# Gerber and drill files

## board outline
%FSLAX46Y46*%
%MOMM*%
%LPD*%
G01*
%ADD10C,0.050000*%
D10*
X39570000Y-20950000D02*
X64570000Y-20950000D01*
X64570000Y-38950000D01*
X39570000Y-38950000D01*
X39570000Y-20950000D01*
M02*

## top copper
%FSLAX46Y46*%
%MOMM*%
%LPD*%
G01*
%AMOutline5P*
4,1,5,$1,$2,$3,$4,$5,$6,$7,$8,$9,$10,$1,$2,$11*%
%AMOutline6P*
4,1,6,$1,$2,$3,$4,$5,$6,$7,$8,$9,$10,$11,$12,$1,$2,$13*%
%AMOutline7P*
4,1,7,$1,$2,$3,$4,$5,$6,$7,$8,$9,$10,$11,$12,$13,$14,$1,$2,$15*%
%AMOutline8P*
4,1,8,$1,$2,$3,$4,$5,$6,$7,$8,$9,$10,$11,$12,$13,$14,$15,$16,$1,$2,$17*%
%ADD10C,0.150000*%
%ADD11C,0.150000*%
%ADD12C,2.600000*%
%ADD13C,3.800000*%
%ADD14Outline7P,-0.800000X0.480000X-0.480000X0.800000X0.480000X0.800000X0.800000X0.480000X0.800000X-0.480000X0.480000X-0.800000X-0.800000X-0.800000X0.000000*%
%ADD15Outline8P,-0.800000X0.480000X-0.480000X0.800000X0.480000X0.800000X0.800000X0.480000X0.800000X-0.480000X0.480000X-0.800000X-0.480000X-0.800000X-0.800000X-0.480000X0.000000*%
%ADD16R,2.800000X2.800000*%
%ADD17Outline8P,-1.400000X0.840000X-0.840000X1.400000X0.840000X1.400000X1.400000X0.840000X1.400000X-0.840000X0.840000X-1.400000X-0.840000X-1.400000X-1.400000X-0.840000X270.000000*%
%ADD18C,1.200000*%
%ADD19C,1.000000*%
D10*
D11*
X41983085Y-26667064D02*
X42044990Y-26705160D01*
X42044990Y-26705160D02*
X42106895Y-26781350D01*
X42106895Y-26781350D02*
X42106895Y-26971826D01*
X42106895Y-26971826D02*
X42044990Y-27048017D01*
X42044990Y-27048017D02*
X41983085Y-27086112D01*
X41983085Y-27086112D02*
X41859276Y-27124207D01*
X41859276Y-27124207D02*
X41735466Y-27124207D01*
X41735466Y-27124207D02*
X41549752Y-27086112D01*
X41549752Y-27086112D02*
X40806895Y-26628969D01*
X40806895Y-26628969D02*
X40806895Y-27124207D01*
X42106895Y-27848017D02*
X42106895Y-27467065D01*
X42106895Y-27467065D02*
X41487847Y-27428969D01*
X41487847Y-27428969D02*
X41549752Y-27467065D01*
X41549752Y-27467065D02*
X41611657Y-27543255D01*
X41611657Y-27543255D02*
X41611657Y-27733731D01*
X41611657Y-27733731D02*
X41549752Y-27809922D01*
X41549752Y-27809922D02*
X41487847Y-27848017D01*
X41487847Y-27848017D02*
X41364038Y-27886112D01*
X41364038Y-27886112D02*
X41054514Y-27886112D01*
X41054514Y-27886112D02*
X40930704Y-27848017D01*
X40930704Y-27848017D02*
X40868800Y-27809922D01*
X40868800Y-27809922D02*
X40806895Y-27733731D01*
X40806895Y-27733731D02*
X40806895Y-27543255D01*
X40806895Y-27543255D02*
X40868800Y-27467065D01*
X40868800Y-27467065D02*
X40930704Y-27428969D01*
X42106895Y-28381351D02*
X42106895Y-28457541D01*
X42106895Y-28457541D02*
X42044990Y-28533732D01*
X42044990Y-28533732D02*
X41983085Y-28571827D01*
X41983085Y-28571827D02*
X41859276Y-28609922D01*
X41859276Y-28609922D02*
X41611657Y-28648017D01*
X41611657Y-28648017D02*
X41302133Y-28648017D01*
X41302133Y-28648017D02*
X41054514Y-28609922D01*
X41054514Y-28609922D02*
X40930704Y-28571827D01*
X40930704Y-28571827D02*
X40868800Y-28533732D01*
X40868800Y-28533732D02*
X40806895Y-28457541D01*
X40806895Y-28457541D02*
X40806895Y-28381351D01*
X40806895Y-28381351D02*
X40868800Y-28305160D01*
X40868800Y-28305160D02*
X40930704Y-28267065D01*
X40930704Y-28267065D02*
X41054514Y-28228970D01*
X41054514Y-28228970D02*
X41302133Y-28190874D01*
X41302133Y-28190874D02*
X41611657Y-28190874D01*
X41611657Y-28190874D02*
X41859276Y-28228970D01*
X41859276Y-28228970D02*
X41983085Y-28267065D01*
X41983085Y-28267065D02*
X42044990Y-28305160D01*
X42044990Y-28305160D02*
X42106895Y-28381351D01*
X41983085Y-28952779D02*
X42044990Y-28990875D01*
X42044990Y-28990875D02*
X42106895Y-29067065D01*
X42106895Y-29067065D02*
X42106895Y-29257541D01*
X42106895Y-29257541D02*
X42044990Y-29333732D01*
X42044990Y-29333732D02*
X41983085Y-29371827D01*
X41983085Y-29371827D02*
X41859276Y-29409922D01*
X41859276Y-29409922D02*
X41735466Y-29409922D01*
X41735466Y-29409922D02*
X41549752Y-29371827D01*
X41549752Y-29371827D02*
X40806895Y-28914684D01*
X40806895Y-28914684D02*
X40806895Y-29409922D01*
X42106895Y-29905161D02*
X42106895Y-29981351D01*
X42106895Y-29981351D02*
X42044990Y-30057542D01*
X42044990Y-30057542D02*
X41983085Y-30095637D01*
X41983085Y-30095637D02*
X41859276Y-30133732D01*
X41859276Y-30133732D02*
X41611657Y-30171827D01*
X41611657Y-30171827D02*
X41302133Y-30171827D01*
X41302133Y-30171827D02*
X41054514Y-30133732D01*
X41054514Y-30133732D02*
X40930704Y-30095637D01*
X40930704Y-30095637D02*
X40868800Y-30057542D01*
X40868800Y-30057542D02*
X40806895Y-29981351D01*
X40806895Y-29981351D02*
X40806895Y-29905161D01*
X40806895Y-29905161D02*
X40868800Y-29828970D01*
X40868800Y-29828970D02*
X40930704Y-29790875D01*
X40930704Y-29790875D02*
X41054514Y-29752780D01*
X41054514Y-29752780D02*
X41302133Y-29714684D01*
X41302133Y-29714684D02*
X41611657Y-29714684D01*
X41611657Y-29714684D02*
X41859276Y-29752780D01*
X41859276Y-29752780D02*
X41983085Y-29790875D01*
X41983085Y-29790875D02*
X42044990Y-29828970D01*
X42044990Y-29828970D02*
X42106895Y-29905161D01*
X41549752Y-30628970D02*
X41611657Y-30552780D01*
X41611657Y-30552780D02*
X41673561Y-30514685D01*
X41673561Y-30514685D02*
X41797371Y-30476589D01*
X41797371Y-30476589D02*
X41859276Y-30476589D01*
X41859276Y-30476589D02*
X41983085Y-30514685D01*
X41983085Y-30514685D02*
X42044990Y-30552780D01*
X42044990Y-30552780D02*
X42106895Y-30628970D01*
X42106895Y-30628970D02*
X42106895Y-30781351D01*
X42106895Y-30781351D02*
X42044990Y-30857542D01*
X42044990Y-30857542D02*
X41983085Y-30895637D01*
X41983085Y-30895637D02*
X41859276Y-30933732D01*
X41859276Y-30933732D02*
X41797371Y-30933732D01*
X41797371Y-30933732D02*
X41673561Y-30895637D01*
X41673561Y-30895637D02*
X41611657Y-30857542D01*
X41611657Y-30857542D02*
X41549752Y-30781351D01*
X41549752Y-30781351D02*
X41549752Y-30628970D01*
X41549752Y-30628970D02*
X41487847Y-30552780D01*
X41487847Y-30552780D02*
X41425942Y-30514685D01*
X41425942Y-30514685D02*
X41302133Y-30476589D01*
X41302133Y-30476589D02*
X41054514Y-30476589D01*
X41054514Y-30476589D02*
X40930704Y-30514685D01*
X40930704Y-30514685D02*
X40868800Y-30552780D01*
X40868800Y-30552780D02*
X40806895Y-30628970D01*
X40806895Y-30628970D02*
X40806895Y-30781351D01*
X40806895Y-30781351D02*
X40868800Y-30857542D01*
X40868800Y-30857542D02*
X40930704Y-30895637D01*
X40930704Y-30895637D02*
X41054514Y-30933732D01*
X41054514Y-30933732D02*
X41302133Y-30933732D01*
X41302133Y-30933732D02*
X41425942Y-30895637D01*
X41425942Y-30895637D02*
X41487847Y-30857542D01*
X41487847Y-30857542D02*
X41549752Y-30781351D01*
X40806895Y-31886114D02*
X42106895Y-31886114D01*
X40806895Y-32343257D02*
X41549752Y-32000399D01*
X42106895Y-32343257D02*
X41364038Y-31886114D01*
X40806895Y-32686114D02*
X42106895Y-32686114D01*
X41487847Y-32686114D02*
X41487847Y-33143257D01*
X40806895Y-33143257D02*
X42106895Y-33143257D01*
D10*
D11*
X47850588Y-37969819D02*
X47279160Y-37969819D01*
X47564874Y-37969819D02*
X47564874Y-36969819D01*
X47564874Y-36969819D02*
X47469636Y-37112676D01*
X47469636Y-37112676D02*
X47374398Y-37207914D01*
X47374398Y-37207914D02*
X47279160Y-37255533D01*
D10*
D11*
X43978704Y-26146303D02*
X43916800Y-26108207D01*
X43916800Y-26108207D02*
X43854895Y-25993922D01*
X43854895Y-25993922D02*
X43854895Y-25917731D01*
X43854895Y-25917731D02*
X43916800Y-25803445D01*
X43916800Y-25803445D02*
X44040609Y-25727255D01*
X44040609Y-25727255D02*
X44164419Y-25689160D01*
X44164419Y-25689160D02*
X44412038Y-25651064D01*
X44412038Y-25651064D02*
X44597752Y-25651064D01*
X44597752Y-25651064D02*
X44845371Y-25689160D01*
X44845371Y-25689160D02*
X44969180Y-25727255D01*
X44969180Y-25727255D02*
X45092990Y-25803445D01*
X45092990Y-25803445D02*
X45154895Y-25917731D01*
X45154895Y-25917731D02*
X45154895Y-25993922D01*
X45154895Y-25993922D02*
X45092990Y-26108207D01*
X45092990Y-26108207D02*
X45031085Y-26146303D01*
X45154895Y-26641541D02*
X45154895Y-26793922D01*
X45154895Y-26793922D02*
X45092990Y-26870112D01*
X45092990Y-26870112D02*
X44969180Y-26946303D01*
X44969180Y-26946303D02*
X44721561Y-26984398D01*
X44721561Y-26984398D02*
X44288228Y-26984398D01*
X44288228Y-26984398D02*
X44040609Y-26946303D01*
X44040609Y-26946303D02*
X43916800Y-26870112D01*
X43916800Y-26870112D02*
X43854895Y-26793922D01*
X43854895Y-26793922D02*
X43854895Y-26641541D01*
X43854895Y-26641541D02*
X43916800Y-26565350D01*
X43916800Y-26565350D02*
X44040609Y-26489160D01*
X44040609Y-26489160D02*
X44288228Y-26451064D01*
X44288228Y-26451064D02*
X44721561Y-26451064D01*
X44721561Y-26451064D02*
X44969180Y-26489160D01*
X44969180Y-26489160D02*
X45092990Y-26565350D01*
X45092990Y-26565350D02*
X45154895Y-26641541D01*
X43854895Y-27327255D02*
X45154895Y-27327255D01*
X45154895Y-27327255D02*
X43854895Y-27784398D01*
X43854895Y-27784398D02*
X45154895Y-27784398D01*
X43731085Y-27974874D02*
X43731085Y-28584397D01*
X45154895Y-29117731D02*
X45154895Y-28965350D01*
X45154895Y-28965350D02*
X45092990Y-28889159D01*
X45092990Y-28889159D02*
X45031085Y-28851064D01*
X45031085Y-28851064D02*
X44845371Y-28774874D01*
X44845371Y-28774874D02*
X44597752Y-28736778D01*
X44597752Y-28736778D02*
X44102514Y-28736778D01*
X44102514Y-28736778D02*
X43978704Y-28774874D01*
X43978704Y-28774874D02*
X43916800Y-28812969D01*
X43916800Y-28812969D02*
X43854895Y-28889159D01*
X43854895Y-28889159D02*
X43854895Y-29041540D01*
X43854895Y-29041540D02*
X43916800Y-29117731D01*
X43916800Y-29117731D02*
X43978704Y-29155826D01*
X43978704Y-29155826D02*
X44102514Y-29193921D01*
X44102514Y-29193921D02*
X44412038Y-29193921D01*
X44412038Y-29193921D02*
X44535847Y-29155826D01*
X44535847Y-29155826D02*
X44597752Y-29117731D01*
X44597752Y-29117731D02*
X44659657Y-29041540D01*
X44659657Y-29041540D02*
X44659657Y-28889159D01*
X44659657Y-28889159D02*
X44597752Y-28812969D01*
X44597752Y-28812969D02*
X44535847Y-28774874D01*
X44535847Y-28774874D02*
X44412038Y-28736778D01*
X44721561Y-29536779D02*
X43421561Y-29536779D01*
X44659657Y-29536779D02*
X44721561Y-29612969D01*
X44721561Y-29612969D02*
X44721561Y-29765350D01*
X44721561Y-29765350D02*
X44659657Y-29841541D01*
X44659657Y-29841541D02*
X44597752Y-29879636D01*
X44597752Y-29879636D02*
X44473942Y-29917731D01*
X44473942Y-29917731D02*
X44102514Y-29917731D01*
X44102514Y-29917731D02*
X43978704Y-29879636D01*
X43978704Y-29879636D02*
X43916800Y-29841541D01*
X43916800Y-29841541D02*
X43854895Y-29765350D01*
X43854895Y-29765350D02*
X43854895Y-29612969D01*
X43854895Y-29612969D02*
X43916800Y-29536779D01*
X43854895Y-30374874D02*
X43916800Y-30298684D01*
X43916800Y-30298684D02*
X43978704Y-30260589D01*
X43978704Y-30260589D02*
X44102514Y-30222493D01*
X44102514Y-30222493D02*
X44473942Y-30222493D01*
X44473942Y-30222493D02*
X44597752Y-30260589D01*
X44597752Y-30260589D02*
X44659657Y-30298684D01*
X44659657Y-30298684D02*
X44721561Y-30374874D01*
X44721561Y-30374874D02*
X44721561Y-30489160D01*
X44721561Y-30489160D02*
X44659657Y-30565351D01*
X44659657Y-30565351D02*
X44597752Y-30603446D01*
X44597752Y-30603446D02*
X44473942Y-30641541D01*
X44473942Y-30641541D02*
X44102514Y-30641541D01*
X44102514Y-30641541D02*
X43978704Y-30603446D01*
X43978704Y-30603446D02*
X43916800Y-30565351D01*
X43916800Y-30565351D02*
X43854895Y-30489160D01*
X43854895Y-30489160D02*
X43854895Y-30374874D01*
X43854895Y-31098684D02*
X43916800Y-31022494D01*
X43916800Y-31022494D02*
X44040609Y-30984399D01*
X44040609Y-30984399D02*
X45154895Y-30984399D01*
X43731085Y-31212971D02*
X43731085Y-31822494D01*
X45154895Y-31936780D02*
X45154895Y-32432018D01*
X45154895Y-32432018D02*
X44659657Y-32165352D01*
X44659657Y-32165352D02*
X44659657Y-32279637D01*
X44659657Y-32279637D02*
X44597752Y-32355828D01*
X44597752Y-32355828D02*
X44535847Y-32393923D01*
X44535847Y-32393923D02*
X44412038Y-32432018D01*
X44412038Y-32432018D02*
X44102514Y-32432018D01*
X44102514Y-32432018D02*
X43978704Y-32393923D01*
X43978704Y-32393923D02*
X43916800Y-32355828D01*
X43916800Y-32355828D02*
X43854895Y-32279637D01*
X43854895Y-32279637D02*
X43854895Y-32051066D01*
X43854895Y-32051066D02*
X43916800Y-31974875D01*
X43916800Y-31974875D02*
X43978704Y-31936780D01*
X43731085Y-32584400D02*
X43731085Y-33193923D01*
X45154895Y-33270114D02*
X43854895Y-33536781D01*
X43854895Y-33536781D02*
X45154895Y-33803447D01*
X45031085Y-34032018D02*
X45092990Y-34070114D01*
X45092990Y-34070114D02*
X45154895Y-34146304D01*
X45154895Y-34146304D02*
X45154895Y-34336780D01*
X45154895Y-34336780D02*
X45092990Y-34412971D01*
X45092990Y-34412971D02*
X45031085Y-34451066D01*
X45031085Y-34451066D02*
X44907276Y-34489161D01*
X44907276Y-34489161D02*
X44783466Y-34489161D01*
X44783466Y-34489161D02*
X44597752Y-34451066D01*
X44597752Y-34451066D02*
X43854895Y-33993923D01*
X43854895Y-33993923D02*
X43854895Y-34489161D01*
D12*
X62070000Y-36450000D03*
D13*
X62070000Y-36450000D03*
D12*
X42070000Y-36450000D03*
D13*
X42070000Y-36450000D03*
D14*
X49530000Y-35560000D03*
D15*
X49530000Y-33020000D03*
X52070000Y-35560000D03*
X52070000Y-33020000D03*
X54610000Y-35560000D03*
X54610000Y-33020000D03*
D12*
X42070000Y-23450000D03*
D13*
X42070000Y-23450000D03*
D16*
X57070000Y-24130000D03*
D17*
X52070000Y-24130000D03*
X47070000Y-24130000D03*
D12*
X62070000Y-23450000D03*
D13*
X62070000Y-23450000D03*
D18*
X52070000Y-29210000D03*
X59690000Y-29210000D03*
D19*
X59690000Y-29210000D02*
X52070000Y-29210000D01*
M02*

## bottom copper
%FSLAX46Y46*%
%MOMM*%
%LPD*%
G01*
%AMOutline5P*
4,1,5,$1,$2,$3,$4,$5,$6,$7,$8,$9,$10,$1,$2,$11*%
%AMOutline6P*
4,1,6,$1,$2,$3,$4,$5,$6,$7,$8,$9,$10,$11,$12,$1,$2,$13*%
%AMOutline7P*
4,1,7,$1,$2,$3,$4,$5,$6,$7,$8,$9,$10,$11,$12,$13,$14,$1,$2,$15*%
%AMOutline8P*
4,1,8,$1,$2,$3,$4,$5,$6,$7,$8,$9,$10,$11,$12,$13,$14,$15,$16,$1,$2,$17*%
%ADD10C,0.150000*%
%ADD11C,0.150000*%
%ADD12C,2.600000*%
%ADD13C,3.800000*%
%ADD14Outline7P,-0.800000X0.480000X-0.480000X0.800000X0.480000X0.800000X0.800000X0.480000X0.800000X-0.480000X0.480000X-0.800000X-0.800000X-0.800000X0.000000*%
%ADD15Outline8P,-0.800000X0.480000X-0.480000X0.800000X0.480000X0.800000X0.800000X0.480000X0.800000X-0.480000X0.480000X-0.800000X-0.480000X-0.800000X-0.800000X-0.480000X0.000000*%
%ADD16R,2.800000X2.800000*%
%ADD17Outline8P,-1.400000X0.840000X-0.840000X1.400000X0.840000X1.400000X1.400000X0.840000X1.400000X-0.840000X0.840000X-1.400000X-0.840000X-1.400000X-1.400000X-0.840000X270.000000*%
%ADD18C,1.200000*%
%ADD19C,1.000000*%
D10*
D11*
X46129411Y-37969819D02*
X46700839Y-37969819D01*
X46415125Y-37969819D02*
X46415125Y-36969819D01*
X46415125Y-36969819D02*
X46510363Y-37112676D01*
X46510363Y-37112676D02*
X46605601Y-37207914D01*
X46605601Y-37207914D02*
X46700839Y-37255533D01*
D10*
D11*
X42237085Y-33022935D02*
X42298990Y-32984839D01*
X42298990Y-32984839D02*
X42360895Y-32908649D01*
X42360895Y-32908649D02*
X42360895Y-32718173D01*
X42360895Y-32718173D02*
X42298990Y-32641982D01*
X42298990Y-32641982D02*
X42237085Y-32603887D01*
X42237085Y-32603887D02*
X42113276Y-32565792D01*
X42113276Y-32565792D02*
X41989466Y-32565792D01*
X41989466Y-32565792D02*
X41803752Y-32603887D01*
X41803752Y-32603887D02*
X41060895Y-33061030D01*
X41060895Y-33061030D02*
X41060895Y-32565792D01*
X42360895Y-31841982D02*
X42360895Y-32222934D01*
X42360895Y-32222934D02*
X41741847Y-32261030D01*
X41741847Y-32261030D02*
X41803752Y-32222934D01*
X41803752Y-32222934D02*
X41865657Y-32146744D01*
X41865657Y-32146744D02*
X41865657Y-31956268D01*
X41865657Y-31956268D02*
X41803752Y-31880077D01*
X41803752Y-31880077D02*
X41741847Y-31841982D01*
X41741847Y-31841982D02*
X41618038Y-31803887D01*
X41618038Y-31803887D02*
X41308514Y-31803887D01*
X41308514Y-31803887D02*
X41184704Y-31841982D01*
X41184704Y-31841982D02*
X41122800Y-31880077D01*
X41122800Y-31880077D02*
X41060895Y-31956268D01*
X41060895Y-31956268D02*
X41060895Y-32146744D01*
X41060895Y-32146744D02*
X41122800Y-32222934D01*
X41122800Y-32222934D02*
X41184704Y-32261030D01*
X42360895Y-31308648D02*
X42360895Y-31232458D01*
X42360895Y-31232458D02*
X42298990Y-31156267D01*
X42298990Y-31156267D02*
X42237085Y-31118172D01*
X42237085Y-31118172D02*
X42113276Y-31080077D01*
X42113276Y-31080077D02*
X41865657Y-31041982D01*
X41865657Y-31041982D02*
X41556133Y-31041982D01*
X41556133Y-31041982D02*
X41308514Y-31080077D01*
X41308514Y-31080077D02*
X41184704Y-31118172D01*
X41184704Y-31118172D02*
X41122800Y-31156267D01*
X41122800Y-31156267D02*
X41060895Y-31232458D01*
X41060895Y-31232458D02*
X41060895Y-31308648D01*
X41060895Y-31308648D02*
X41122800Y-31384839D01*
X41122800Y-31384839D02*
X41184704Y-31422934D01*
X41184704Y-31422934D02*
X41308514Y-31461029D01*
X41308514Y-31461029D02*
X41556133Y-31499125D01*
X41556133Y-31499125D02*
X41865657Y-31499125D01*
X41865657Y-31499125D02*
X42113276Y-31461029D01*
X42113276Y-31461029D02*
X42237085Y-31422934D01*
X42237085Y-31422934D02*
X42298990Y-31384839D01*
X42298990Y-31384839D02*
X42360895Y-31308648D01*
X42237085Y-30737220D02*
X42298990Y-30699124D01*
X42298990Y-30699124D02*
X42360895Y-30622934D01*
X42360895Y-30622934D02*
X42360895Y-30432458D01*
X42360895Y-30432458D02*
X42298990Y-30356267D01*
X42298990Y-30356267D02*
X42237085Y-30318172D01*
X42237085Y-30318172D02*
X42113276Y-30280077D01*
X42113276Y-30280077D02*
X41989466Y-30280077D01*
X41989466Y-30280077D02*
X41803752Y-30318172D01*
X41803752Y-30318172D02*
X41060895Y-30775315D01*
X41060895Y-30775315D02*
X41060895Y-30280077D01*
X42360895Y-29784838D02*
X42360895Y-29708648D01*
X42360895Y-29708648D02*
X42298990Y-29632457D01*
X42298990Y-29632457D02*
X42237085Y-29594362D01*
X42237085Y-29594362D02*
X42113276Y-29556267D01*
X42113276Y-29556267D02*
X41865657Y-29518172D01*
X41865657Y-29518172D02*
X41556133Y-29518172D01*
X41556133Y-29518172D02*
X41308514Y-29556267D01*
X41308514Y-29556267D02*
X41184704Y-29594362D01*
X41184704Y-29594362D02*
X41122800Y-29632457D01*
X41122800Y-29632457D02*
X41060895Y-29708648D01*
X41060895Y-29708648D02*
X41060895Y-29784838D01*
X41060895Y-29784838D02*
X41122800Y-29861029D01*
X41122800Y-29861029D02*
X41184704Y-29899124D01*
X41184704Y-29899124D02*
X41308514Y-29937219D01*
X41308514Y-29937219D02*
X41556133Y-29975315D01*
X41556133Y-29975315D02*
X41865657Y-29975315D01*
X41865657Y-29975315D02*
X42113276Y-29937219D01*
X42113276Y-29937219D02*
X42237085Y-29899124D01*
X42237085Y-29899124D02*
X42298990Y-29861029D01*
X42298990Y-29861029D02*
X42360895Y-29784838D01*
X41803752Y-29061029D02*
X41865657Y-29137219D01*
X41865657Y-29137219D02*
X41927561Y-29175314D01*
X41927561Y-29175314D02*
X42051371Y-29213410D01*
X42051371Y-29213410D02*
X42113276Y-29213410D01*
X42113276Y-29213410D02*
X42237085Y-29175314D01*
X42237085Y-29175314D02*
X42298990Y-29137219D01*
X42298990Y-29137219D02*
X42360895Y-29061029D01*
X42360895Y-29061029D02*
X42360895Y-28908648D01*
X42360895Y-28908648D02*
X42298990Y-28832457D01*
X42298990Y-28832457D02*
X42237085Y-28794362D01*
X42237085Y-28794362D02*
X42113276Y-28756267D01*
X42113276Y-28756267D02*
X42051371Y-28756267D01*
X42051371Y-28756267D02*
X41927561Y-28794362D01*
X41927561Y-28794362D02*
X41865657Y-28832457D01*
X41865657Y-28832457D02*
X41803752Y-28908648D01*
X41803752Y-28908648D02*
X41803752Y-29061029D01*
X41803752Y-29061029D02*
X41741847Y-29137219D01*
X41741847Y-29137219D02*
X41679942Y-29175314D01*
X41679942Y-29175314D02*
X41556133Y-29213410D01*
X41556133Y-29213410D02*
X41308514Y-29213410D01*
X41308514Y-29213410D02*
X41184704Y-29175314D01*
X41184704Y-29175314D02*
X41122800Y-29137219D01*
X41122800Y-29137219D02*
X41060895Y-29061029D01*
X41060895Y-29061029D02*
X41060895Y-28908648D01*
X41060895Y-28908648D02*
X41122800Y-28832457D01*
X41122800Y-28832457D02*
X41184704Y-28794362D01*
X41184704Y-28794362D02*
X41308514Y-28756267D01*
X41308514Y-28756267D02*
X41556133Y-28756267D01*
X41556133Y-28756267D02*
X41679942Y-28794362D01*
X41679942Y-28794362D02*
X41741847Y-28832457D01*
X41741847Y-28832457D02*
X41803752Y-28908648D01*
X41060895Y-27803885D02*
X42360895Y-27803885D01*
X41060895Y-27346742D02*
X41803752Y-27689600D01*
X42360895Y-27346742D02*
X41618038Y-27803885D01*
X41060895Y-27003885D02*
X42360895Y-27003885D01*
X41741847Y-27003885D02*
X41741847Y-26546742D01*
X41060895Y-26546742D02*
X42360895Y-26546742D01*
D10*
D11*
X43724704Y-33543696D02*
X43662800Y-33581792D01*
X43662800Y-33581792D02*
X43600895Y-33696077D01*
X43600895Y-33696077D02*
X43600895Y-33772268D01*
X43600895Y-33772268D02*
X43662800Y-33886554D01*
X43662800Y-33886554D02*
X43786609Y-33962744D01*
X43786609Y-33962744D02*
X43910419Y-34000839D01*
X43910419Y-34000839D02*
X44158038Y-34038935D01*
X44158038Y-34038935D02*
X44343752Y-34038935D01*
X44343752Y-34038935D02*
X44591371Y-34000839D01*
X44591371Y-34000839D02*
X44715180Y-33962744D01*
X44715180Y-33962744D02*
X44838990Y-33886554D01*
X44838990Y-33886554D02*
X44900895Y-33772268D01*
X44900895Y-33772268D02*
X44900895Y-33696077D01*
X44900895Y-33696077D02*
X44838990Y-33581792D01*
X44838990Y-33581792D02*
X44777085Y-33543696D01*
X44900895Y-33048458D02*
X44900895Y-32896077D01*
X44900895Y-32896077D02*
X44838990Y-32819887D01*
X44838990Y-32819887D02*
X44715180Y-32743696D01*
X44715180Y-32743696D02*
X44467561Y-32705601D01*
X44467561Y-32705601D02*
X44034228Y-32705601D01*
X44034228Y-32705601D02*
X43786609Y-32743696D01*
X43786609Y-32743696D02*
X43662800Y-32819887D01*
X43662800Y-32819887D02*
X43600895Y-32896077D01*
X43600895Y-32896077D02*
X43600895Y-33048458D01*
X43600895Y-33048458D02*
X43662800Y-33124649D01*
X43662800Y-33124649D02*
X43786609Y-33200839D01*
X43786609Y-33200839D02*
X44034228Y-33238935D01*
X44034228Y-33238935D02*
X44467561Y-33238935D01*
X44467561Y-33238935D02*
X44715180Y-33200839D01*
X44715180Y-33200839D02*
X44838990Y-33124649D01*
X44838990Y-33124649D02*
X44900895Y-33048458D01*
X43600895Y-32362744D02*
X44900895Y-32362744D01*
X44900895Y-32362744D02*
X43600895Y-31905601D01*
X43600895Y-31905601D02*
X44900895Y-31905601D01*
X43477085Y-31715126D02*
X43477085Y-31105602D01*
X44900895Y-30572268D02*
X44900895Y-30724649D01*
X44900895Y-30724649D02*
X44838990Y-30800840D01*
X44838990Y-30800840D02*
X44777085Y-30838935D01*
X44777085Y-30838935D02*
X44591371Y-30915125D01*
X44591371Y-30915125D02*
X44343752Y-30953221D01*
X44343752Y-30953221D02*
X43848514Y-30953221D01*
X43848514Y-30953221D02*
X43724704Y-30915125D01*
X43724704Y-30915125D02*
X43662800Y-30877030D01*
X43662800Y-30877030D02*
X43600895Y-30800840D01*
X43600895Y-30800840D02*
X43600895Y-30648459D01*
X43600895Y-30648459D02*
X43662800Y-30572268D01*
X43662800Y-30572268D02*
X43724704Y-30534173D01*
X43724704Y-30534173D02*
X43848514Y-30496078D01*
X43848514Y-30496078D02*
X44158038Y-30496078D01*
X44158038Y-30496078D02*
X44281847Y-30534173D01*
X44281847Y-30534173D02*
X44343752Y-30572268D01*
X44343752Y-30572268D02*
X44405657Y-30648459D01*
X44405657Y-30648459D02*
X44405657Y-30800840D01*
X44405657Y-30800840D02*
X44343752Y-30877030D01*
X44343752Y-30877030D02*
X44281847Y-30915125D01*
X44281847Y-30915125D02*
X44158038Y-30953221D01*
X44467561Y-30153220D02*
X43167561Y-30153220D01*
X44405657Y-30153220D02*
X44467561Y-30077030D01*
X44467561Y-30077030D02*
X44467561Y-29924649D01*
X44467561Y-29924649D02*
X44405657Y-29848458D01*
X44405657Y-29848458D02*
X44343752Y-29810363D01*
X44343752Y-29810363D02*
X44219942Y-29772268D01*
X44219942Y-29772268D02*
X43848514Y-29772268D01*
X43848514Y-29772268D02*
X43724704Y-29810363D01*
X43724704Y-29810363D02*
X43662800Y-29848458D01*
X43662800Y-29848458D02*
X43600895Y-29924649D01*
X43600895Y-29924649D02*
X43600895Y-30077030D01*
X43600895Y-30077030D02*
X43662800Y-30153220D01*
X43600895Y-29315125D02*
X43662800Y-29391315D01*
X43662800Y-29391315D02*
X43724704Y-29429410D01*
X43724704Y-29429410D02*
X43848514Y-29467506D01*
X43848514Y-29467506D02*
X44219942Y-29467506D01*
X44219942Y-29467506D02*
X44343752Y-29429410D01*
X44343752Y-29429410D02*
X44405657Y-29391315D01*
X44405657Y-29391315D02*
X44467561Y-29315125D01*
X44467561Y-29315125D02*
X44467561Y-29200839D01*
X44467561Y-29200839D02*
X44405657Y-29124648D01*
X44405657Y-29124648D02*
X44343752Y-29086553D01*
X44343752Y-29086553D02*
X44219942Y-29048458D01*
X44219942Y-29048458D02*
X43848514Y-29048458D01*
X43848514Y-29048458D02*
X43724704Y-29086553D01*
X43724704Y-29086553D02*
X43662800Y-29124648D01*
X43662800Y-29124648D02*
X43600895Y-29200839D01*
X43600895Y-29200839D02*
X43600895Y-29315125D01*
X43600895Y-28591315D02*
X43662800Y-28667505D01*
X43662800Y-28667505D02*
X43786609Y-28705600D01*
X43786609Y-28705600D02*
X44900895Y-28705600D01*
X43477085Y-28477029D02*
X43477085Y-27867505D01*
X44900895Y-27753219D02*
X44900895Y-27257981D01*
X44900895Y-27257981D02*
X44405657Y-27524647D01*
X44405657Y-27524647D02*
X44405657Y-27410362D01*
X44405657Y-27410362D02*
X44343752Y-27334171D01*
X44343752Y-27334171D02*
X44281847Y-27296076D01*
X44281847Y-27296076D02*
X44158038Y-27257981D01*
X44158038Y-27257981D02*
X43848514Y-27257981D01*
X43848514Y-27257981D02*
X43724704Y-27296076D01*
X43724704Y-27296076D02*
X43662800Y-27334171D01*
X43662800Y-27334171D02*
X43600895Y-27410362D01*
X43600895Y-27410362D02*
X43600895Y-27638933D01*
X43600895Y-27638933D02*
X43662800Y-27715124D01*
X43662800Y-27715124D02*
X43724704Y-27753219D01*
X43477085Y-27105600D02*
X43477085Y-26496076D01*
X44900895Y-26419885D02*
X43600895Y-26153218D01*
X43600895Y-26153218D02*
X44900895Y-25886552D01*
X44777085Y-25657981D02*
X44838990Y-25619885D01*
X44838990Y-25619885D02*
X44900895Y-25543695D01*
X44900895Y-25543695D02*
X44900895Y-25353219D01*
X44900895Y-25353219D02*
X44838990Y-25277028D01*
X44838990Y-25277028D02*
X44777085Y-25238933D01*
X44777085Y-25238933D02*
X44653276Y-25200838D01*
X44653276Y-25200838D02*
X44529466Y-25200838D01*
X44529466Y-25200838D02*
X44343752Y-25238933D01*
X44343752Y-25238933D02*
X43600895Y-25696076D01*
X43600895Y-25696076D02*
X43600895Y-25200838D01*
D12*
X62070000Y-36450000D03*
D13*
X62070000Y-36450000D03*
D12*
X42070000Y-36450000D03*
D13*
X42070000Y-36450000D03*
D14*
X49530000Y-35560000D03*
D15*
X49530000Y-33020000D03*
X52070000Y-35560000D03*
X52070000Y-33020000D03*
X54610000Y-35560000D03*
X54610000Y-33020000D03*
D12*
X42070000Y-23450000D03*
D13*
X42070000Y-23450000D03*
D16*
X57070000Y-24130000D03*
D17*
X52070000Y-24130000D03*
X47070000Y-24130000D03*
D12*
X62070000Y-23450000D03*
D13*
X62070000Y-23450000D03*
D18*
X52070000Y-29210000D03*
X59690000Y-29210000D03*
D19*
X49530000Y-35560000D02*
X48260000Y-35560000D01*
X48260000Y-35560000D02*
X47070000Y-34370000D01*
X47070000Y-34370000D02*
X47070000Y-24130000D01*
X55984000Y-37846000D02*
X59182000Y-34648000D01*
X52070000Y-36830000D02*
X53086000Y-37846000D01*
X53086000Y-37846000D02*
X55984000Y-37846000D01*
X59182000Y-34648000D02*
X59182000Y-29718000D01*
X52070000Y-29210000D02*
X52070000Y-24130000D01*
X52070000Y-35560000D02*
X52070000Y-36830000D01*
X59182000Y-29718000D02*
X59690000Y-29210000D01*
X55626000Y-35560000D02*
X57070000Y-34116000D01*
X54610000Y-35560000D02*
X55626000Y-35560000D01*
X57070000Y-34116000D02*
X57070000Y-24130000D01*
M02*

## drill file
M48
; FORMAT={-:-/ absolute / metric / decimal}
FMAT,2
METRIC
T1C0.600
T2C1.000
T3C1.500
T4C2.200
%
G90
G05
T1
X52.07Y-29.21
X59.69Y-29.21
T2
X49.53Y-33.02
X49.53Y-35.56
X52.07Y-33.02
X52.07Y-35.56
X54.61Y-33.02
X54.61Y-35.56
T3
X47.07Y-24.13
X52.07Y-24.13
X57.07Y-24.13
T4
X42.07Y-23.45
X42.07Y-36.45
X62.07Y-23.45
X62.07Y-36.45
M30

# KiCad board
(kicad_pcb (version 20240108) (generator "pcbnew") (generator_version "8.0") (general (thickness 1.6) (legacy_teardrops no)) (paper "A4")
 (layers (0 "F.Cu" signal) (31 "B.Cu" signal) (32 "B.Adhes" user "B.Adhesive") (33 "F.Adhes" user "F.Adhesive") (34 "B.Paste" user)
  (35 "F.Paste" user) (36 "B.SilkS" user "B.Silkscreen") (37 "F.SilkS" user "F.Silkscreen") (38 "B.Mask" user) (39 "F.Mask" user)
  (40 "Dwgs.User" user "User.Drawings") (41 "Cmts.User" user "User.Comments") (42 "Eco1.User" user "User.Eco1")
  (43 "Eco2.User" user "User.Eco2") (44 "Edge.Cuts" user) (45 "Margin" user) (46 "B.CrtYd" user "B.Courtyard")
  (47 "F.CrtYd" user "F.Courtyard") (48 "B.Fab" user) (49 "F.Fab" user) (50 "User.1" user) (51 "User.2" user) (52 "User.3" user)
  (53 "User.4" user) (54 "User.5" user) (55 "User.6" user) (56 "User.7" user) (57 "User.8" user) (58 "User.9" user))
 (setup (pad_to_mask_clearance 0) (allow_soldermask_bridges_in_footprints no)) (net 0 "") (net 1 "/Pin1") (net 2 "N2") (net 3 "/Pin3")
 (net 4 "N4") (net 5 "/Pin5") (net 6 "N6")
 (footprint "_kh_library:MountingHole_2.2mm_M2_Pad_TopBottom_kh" (layer "F.Cu") (at 62.07 36.45)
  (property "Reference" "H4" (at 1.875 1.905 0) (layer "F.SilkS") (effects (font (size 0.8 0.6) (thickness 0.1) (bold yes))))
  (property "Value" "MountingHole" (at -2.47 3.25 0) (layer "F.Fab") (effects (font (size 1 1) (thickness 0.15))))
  (pad "1" thru_hole circle (at 0 0) (size 2.6 2.6) (drill 2.2) (layers "*.Cu" "*.Mask") (remove_unused_layers no))
  (pad "1" connect circle (at 0 0) (size 3.8 3.8) (layers "F.Cu" "F.Mask"))
  (pad "1" connect circle (at 0 0) (size 3.8 3.8) (layers "B.Cu" "B.Mask")))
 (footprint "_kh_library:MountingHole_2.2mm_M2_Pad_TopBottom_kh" (layer "F.Cu") (at 42.07 36.45)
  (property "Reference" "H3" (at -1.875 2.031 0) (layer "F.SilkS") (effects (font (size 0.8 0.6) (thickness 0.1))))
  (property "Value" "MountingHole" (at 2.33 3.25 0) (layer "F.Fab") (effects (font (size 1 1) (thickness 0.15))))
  (pad "1" thru_hole circle (at 0 0) (size 2.6 2.6) (drill 2.2) (layers "*.Cu" "*.Mask") (remove_unused_layers no))
  (pad "1" connect circle (at 0 0) (size 3.8 3.8) (layers "F.Cu" "F.Mask"))
  (pad "1" connect circle (at 0 0) (size 3.8 3.8) (layers "B.Cu" "B.Mask")))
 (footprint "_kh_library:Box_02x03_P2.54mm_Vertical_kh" (layer "F.Cu") (at 49.53 35.56)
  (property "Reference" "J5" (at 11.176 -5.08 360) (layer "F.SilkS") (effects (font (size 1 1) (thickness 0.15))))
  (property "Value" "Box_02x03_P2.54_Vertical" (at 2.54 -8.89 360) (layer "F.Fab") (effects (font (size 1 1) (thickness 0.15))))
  (pad "1" thru_hole roundrect (at 0 0) (size 1.6 1.6) (drill 1) (layers "*.Cu" "*.Mask") (remove_unused_layers no) (roundrect_rratio 0)
   (chamfer_ratio 0.2) (chamfer top_left top_right bottom_right) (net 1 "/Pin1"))
  (pad "2" thru_hole roundrect (at 0 -2.54) (size 1.6 1.6) (drill 1) (layers "*.Cu" "*.Mask") (remove_unused_layers no) (roundrect_rratio 0)
   (chamfer_ratio 0.2) (chamfer top_left top_right bottom_left bottom_right) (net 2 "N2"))
  (pad "3" thru_hole roundrect (at 2.54 0) (size 1.6 1.6) (drill 1) (layers "*.Cu" "*.Mask") (remove_unused_layers no) (roundrect_rratio 0)
   (chamfer_ratio 0.2) (chamfer top_left top_right bottom_left bottom_right) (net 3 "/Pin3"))
  (pad "4" thru_hole roundrect (at 2.54 -2.54) (size 1.6 1.6) (drill 1) (layers "*.Cu" "*.Mask") (remove_unused_layers no)
   (roundrect_rratio 0) (chamfer_ratio 0.2) (chamfer top_left top_right bottom_left bottom_right) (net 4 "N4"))
  (pad "5" thru_hole roundrect (at 5.08 0) (size 1.6 1.6) (drill 1) (layers "*.Cu" "*.Mask") (remove_unused_layers no) (roundrect_rratio 0)
   (chamfer_ratio 0.2) (chamfer top_left top_right bottom_left bottom_right) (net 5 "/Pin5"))
  (pad "6" thru_hole roundrect (at 5.08 -2.54) (size 1.6 1.6) (drill 1) (layers "*.Cu" "*.Mask") (remove_unused_layers no)
   (roundrect_rratio 0) (chamfer_ratio 0.2) (chamfer top_left top_right bottom_left bottom_right) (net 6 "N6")))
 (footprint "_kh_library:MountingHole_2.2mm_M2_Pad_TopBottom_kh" (layer "F.Cu") (at 42.07 23.45)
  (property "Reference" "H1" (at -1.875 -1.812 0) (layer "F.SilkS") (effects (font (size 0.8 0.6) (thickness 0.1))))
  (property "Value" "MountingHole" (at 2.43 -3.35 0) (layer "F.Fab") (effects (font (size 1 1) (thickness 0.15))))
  (pad "1" thru_hole circle (at 0 0) (size 2.6 2.6) (drill 2.2) (layers "*.Cu" "*.Mask") (remove_unused_layers no))
  (pad "1" connect circle (at 0 0) (size 3.8 3.8) (layers "F.Cu" "F.Mask"))
  (pad "1" connect circle (at 0 0) (size 3.8 3.8) (layers "B.Cu" "B.Mask")))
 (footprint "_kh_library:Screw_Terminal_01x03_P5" (layer "F.Cu") (at 57.07 24.13 -90)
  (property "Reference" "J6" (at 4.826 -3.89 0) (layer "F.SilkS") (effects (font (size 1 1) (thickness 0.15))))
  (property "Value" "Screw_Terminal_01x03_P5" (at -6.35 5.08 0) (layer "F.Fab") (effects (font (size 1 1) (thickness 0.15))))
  (pad "1" thru_hole rect (at 0 0 270) (size 2.8 2.8) (drill 1.5) (layers "*.Cu" "*.Mask") (remove_unused_layers no) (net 5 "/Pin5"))
  (pad "2" thru_hole roundrect (at 0 5 270) (size 2.8 2.8) (drill 1.5) (layers "*.Cu" "*.Mask") (remove_unused_layers no)
   (roundrect_rratio 0) (chamfer_ratio 0.2) (chamfer top_left top_right bottom_left bottom_right) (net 3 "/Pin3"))
  (pad "3" thru_hole roundrect (at 0 10 270) (size 2.8 2.8) (drill 1.5) (layers "*.Cu" "*.Mask") (remove_unused_layers no)
   (roundrect_rratio 0) (chamfer_ratio 0.2) (chamfer top_left top_right bottom_left bottom_right) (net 1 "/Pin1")))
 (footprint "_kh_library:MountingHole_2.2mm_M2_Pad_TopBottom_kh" (layer "F.Cu") (at 62.07 23.45)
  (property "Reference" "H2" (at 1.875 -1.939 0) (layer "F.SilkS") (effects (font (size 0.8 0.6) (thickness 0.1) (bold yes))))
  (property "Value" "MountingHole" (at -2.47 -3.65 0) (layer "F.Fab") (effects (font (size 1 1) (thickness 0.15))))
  (pad "1" thru_hole circle (at 0 0) (size 2.6 2.6) (drill 2.2) (layers "*.Cu" "*.Mask") (remove_unused_layers no))
  (pad "1" connect circle (at 0 0) (size 3.8 3.8) (layers "F.Cu" "F.Mask"))
  (pad "1" connect circle (at 0 0) (size 3.8 3.8) (layers "B.Cu" "B.Mask")))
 (gr_rect (start 39.57 20.95) (end 64.57 38.95) (stroke (width 0.05) (type default)) (fill none) (layer "Edge.Cuts"))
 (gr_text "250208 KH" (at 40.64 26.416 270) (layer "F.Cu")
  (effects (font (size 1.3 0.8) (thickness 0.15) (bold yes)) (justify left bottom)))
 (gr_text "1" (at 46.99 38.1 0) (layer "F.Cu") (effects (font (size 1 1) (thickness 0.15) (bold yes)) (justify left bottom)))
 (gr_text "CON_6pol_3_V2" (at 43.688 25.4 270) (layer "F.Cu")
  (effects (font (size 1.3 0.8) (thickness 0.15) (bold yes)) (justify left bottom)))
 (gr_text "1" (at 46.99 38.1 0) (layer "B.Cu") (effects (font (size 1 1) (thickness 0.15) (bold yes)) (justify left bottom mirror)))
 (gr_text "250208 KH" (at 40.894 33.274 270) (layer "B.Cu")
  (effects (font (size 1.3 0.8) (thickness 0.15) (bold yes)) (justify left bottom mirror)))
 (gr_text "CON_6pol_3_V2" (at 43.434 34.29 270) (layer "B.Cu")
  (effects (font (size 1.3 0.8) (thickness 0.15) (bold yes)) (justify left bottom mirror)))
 (segment (start 49.53 35.56) (end 48.26 35.56) (width 1) (layer "B.Cu") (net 1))
 (segment (start 48.26 35.56) (end 47.07 34.37) (width 1) (layer "B.Cu") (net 1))
 (segment (start 47.07 34.37) (end 47.07 24.13) (width 1) (layer "B.Cu") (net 1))
 (segment (start 59.69 29.21) (end 52.07 29.21) (width 1) (layer "F.Cu") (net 3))
 (via (at 52.07 29.21) (size 1.2) (drill 0.6) (layers "F.Cu" "B.Cu") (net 3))
 (via (at 59.69 29.21) (size 1.2) (drill 0.6) (layers "F.Cu" "B.Cu") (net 3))
 (segment (start 55.984 37.846) (end 59.182 34.648) (width 1) (layer "B.Cu") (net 3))
 (segment (start 52.07 36.83) (end 53.086 37.846) (width 1) (layer "B.Cu") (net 3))
 (segment (start 53.086 37.846) (end 55.984 37.846) (width 1) (layer "B.Cu") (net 3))
 (segment (start 59.182 34.648) (end 59.182 29.718) (width 1) (layer "B.Cu") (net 3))
 (segment (start 52.07 29.21) (end 52.07 24.13) (width 1) (layer "B.Cu") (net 3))
 (segment (start 52.07 35.56) (end 52.07 36.83) (width 1) (layer "B.Cu") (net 3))
 (segment (start 59.182 29.718) (end 59.69 29.21) (width 1) (layer "B.Cu") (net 3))
 (segment (start 55.626 35.56) (end 57.07 34.116) (width 1) (layer "B.Cu") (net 5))
 (segment (start 54.61 35.56) (end 55.626 35.56) (width 1) (layer "B.Cu") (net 5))
 (segment (start 57.07 34.116) (end 57.07 24.13) (width 1) (layer "B.Cu") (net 5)))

